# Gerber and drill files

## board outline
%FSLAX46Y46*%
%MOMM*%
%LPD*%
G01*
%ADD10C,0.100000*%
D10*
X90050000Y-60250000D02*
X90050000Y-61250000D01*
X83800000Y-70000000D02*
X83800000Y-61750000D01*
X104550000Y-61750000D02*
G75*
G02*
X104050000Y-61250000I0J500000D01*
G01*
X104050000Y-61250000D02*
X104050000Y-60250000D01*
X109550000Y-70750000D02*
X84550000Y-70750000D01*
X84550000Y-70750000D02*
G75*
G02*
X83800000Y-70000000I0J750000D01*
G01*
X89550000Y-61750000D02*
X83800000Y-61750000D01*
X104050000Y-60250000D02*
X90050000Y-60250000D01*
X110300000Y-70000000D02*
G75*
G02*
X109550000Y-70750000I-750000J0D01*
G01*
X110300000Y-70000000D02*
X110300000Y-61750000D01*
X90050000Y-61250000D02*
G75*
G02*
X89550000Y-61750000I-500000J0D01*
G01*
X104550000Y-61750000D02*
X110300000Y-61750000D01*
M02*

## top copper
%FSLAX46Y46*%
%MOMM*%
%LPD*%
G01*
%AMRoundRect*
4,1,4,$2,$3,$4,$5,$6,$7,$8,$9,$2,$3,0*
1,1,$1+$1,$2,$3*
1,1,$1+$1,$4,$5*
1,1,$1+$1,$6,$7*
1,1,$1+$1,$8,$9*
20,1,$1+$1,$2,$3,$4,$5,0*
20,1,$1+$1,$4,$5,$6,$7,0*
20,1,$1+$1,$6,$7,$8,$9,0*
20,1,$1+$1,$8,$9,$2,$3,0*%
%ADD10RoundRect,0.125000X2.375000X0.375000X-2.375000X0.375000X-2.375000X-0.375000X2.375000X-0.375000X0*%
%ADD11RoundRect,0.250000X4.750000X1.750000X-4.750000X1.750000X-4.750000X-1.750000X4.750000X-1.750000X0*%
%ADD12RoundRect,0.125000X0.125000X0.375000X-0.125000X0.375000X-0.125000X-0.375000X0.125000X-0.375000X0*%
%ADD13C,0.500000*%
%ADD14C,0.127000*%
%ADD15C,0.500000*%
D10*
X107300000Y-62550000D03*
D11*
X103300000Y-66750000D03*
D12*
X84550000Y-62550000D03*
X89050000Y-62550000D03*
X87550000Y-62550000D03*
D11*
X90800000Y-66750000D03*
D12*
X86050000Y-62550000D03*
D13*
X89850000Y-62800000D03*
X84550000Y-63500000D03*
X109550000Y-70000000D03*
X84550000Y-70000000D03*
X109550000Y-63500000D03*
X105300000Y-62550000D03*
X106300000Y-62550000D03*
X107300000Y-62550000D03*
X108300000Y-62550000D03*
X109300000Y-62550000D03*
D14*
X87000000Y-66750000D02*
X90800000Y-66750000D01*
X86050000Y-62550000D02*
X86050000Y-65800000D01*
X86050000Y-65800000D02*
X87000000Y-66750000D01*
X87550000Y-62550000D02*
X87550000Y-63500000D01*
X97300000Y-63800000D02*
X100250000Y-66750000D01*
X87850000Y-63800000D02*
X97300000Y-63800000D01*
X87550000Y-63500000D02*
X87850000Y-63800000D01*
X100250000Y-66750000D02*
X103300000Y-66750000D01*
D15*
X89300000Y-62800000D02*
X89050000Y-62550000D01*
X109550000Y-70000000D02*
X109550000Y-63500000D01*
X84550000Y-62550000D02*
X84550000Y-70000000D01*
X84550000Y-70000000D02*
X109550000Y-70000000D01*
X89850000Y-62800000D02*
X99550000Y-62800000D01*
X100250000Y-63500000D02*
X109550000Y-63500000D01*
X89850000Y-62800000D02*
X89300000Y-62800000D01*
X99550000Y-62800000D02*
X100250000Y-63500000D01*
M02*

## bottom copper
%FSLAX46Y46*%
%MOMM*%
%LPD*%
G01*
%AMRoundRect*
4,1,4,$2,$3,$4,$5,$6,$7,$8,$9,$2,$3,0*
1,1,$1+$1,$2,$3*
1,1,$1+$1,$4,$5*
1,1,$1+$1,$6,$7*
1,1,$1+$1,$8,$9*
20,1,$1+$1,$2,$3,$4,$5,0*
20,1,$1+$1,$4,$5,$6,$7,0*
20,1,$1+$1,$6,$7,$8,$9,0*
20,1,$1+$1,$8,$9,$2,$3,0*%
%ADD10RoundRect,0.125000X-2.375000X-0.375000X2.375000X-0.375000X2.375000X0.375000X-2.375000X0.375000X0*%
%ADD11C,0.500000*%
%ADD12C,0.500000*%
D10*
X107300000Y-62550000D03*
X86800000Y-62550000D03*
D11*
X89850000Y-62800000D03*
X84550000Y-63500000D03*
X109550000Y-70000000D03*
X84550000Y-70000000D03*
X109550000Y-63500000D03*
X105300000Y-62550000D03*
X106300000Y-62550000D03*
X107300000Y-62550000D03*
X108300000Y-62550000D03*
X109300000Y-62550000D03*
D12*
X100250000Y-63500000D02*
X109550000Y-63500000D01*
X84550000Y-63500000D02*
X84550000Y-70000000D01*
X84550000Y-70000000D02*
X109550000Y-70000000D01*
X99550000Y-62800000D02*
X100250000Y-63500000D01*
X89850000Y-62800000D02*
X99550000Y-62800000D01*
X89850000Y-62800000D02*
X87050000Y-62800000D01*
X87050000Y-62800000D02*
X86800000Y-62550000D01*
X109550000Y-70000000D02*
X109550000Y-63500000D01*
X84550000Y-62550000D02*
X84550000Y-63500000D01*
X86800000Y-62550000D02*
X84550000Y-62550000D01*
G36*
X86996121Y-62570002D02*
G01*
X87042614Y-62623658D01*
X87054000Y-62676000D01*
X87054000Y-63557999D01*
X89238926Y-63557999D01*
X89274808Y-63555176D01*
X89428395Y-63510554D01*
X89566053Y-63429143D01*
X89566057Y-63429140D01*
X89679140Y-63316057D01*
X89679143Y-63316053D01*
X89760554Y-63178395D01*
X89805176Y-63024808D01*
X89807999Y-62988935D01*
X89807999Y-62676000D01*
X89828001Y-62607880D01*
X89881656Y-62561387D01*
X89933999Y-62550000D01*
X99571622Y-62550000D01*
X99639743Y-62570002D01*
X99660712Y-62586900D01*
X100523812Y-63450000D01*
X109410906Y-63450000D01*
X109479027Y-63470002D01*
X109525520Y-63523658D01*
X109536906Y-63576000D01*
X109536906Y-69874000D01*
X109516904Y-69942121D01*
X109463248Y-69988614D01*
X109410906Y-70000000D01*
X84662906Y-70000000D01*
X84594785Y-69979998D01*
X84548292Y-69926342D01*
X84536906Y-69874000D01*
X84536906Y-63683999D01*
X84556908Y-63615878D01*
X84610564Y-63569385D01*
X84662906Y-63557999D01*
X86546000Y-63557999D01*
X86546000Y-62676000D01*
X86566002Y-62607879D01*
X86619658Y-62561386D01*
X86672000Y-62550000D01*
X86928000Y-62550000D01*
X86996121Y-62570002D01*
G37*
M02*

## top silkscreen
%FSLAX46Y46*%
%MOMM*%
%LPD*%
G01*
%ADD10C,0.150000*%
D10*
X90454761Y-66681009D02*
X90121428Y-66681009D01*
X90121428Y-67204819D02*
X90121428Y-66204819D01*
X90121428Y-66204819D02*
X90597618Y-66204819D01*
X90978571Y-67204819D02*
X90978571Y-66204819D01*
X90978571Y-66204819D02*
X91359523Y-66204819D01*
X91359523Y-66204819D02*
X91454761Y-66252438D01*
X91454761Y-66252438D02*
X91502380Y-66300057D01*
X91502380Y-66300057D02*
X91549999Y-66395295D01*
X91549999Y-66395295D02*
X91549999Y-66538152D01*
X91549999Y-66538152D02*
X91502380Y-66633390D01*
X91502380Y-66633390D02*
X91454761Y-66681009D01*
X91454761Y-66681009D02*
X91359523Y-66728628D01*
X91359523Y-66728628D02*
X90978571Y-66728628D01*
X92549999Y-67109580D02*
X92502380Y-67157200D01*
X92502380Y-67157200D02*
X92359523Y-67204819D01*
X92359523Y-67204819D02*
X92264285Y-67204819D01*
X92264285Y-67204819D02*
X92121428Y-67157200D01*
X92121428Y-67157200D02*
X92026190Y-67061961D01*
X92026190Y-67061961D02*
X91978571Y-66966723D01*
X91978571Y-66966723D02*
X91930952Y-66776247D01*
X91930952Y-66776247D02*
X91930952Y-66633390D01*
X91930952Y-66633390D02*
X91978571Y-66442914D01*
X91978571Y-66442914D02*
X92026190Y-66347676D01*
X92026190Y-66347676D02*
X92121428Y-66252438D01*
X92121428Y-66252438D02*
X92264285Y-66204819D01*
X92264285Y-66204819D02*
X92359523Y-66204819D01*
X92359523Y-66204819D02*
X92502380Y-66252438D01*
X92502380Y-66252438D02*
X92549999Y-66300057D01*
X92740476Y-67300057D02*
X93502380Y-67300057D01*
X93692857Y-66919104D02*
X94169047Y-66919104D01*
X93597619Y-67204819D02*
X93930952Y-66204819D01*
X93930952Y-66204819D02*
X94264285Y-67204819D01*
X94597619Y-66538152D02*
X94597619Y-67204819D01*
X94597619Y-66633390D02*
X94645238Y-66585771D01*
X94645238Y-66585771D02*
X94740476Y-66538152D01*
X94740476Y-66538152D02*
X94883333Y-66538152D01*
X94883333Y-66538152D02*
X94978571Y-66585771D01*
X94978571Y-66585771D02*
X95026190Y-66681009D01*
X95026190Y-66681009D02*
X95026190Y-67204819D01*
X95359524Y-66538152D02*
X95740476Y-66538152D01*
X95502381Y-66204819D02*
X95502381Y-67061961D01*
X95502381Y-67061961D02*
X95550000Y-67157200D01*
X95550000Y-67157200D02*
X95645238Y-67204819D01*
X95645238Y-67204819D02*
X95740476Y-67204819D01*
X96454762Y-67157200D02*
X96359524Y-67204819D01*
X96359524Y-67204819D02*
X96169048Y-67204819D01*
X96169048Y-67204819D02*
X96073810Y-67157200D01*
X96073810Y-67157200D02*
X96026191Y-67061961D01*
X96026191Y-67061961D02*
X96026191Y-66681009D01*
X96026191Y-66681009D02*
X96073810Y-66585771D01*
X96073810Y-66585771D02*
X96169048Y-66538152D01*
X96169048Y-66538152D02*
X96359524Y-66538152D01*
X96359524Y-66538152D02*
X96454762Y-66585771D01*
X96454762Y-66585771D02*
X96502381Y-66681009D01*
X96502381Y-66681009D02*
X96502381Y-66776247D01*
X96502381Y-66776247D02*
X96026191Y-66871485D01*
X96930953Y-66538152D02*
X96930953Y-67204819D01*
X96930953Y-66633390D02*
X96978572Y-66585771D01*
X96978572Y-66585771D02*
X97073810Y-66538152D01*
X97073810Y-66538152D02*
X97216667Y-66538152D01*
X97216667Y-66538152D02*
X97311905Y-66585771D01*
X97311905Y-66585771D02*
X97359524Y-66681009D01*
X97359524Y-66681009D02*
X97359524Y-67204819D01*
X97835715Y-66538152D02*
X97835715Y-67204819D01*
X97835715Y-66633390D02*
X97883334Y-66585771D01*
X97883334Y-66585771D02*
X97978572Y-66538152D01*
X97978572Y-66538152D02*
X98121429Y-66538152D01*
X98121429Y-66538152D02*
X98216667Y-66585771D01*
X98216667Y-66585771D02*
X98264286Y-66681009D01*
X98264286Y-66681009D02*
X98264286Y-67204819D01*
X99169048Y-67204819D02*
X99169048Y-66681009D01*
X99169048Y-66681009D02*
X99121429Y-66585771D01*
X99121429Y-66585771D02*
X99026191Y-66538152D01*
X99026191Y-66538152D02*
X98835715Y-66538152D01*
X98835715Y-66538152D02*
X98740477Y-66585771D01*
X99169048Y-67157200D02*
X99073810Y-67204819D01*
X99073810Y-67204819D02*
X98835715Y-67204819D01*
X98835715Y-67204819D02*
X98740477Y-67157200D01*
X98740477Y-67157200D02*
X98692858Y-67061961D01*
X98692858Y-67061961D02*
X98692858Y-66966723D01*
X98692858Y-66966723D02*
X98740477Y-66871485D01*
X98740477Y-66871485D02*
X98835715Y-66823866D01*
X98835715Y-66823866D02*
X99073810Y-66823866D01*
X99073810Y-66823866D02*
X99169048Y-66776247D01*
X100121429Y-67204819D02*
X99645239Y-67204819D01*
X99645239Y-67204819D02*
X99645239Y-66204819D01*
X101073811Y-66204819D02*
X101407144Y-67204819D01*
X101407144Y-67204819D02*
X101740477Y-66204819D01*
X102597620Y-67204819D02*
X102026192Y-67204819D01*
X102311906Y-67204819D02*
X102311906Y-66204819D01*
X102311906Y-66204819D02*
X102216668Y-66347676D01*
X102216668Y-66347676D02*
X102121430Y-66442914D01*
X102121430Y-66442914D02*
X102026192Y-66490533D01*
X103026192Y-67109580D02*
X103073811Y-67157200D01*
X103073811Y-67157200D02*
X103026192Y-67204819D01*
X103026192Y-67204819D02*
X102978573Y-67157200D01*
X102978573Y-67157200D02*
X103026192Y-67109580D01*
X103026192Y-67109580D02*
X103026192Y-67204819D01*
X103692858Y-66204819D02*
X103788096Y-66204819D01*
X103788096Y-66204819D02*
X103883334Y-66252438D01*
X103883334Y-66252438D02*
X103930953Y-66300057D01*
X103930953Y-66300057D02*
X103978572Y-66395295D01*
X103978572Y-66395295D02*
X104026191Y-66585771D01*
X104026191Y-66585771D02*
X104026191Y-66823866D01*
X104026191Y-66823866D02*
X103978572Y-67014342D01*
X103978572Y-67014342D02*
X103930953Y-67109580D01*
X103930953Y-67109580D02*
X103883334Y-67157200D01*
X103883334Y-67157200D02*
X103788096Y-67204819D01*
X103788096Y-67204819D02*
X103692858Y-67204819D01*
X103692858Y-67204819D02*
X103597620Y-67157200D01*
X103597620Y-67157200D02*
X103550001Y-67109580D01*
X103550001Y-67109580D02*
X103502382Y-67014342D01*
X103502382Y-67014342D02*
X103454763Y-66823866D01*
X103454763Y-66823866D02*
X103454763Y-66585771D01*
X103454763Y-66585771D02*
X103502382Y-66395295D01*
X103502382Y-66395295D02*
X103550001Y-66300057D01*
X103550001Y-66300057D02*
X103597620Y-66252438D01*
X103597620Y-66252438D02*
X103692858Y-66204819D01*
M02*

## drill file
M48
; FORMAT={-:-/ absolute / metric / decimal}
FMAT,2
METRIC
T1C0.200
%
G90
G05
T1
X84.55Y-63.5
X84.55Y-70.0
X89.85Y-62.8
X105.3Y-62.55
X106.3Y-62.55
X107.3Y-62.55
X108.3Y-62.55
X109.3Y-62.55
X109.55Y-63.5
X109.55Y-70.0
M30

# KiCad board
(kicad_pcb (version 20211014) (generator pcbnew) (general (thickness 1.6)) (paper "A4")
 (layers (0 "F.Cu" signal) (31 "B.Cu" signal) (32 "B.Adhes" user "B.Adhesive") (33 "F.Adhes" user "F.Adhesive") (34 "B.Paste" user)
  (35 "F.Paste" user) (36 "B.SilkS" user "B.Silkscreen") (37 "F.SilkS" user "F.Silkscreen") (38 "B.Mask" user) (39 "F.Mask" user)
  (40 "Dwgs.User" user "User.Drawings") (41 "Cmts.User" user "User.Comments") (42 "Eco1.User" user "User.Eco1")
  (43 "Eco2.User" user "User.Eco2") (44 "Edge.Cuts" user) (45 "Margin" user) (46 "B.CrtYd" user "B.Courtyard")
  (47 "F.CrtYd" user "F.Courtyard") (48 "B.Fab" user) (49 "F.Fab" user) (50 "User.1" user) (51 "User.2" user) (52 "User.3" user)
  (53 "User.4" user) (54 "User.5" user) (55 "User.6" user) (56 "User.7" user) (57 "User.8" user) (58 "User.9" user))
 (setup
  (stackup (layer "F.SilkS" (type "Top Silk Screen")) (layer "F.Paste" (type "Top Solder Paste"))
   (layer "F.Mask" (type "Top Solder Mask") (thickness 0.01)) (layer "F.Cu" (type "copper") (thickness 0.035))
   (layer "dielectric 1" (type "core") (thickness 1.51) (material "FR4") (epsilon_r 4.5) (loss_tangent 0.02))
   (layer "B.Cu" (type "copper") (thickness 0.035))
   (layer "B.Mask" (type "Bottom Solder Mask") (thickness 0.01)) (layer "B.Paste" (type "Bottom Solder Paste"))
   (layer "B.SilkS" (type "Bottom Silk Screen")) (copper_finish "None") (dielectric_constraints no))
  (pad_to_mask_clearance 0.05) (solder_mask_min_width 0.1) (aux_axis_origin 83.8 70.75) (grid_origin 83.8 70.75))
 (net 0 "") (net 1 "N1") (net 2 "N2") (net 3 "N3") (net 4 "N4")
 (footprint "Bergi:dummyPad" (layer "F.Cu") (at 107.3 62.55 180)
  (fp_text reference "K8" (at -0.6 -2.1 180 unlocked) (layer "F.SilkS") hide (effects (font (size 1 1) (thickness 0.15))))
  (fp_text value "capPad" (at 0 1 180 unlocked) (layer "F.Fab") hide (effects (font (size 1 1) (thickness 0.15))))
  (pad "1" smd roundrect (at 0 0 180) (size 5 1) (layers "F.Cu" "F.Mask") (roundrect_rratio 0.125) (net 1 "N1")))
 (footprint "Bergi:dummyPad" (layer "F.Cu") (at 103.3 66.75 180)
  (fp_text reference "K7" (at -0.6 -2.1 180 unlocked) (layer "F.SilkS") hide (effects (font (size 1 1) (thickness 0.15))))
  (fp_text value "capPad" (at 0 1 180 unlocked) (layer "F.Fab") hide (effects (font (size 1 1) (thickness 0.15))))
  (pad "1" smd roundrect (at 0 0 180) (size 10 4) (layers "F.Cu") (roundrect_rratio 0.0625) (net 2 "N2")))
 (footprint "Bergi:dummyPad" (layer "F.Cu") (at 84.55 62.55 180)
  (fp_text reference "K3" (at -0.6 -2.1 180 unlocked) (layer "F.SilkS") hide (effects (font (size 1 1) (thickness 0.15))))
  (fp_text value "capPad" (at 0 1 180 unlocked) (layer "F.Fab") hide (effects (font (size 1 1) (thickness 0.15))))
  (pad "1" smd roundrect (at 0 0 180) (size 0.5 1) (layers "F.Cu" "F.Mask") (roundrect_rratio 0.25) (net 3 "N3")))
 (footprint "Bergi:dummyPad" (layer "F.Cu") (at 89.05 62.55 180)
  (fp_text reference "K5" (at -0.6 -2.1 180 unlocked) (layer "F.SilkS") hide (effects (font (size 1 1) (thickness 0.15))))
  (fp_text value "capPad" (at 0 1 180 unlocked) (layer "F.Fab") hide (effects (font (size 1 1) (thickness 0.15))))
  (pad "1" smd roundrect (at 0 0 180) (size 0.5 1) (layers "F.Cu" "F.Mask") (roundrect_rratio 0.25) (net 3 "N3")))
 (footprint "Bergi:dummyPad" (layer "F.Cu") (at 87.55 62.55 180)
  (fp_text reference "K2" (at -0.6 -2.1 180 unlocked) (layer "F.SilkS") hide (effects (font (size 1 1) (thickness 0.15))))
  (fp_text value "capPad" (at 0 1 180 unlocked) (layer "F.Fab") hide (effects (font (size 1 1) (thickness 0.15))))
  (pad "1" smd roundrect (at 0 0 180) (size 0.5 1) (layers "F.Cu" "F.Mask") (roundrect_rratio 0.25) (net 2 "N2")))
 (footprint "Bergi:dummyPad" (layer "F.Cu") (at 90.8 66.75 180)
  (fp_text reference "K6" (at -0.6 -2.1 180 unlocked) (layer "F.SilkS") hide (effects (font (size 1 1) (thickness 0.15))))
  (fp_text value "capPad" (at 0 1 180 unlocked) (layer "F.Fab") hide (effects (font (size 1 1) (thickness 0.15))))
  (pad "1" smd roundrect (at 0 0 180) (size 10 4) (layers "F.Cu") (roundrect_rratio 0.0625) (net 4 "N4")))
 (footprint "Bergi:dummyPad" (layer "F.Cu") (at 86.05 62.55 180)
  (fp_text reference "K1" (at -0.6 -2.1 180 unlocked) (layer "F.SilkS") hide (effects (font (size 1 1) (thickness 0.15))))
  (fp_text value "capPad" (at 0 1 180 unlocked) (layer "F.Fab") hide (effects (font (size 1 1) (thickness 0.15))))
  (pad "1" smd roundrect (at 0 0 180) (size 0.5 1) (layers "F.Cu" "F.Mask") (roundrect_rratio 0.25) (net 4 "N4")))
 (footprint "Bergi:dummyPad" (layer "B.Cu") (at 107.3 62.55)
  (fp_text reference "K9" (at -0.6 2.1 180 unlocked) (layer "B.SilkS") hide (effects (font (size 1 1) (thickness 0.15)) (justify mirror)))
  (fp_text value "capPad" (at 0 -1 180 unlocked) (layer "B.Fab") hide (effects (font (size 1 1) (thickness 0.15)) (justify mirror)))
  (pad "1" smd roundrect (at 0 0) (size 5 1) (layers "B.Cu" "B.Mask") (roundrect_rratio 0.125) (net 1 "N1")))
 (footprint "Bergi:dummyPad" (layer "B.Cu") (at 86.8 62.55)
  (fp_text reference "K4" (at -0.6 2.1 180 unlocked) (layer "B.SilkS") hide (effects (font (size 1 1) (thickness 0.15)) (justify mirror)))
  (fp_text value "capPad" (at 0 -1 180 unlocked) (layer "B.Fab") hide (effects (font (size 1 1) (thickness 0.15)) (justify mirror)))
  (pad "1" smd roundrect (at 0 0) (size 5 1) (layers "B.Cu" "B.Mask") (roundrect_rratio 0.125) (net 3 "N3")))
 (gr_line (start 90.05 60.25) (end 90.05 61.25) (layer "Edge.Cuts") (width 0.1))
 (gr_line (start 83.8 70) (end 83.8 61.75) (layer "Edge.Cuts") (width 0.1))
 (gr_arc (start 104.55 61.75) (mid 104.196447 61.603553) (end 104.05 61.25) (layer "Edge.Cuts") (width 0.1))
 (gr_line (start 104.05 61.25) (end 104.05 60.25) (layer "Edge.Cuts") (width 0.1))
 (gr_line (start 109.55 70.75) (end 84.55 70.75) (layer "Edge.Cuts") (width 0.1))
 (gr_arc (start 84.55 70.75) (mid 84.01967 70.53033) (end 83.8 70) (layer "Edge.Cuts") (width 0.1))
 (gr_line (start 89.55 61.75) (end 83.8 61.75) (layer "Edge.Cuts") (width 0.1))
 (gr_line (start 104.05 60.25) (end 90.05 60.25) (layer "Edge.Cuts") (width 0.1))
 (gr_arc (start 110.3 70) (mid 110.08033 70.53033) (end 109.55 70.75) (layer "Edge.Cuts") (width 0.1))
 (gr_line (start 110.3 70) (end 110.3 61.75) (layer "Edge.Cuts") (width 0.1))
 (gr_arc (start 90.05 61.25) (mid 89.903553 61.603553) (end 89.55 61.75) (layer "Edge.Cuts") (width 0.1))
 (gr_line (start 104.55 61.75) (end 110.3 61.75) (layer "Edge.Cuts") (width 0.1))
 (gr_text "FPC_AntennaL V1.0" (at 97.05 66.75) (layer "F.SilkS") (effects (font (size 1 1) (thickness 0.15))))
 (segment (start 87 66.75) (end 90.8 66.75) (width 0.127) (layer "F.Cu") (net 4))
 (segment (start 86.05 62.55) (end 86.05 65.8) (width 0.127) (layer "F.Cu") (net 4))
 (segment (start 86.05 65.8) (end 87 66.75) (width 0.127) (layer "F.Cu") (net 4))
 (segment (start 87.55 62.55) (end 87.55 63.5) (width 0.127) (layer "F.Cu") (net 2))
 (segment (start 97.3 63.8) (end 100.25 66.75) (width 0.127) (layer "F.Cu") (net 2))
 (segment (start 87.85 63.8) (end 97.3 63.8) (width 0.127) (layer "F.Cu") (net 2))
 (segment (start 87.55 63.5) (end 87.85 63.8) (width 0.127) (layer "F.Cu") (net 2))
 (segment (start 100.25 66.75) (end 103.3 66.75) (width 0.127) (layer "F.Cu") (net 2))
 (segment (start 89.3 62.8) (end 89.05 62.55) (width 0.5) (layer "F.Cu") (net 3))
 (segment (start 109.55 70) (end 109.55 63.5) (width 0.5) (layer "F.Cu") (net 3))
 (segment (start 84.55 62.55) (end 84.55 70) (width 0.5) (layer "F.Cu") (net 3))
 (segment (start 84.55 70) (end 109.55 70) (width 0.5) (layer "F.Cu") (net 3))
 (segment (start 89.85 62.8) (end 99.55 62.8) (width 0.5) (layer "F.Cu") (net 3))
 (segment (start 100.25 63.5) (end 109.55 63.5) (width 0.5) (layer "F.Cu") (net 3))
 (segment (start 89.85 62.8) (end 89.3 62.8) (width 0.5) (layer "F.Cu") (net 3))
 (segment (start 99.55 62.8) (end 100.25 63.5) (width 0.5) (layer "F.Cu") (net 3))
 (via (at 89.85 62.8) (size 0.5) (drill 0.2) (layers "F.Cu" "B.Cu") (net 3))
 (via (at 84.55 63.5) (size 0.5) (drill 0.2) (layers "F.Cu" "B.Cu") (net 3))
 (via (at 109.55 70) (size 0.5) (drill 0.2) (layers "F.Cu" "B.Cu") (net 3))
 (via (at 84.55 70) (size 0.5) (drill 0.2) (layers "F.Cu" "B.Cu") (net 3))
 (via (at 109.55 63.5) (size 0.5) (drill 0.2) (layers "F.Cu" "B.Cu") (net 3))
 (segment (start 100.25 63.5) (end 109.55 63.5) (width 0.5) (layer "B.Cu") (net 3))
 (segment (start 84.55 63.5) (end 84.55 70) (width 0.5) (layer "B.Cu") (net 3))
 (segment (start 84.55 70) (end 109.55 70) (width 0.5) (layer "B.Cu") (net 3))
 (segment (start 99.55 62.8) (end 100.25 63.5) (width 0.5) (layer "B.Cu") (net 3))
 (segment (start 89.85 62.8) (end 99.55 62.8) (width 0.5) (layer "B.Cu") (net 3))
 (segment (start 89.85 62.8) (end 87.05 62.8) (width 0.5) (layer "B.Cu") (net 3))
 (segment (start 87.05 62.8) (end 86.8 62.55) (width 0.5) (layer "B.Cu") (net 3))
 (segment (start 109.55 70) (end 109.55 63.5) (width 0.5) (layer "B.Cu") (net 3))
 (segment (start 84.55 62.55) (end 84.55 63.5) (width 0.5) (layer "B.Cu") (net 3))
 (segment (start 86.8 62.55) (end 84.55 62.55) (width 0.5) (layer "B.Cu") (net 3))
 (via (at 105.3 62.55) (size 0.5) (drill 0.2) (layers "F.Cu" "B.Cu") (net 1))
 (via (at 106.3 62.55) (size 0.5) (drill 0.2) (layers "F.Cu" "B.Cu") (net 1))
 (via (at 107.3 62.55) (size 0.5) (drill 0.2) (layers "F.Cu" "B.Cu") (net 1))
 (via (at 108.3 62.55) (size 0.5) (drill 0.2) (layers "F.Cu" "B.Cu") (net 1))
 (via (at 109.3 62.55) (size 0.5) (drill 0.2) (layers "F.Cu" "B.Cu") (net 1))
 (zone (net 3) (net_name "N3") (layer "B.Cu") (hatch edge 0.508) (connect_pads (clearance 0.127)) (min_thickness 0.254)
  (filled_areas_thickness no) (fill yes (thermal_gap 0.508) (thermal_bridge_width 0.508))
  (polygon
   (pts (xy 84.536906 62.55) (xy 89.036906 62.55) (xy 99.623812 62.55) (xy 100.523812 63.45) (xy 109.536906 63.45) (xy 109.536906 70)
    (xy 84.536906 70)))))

